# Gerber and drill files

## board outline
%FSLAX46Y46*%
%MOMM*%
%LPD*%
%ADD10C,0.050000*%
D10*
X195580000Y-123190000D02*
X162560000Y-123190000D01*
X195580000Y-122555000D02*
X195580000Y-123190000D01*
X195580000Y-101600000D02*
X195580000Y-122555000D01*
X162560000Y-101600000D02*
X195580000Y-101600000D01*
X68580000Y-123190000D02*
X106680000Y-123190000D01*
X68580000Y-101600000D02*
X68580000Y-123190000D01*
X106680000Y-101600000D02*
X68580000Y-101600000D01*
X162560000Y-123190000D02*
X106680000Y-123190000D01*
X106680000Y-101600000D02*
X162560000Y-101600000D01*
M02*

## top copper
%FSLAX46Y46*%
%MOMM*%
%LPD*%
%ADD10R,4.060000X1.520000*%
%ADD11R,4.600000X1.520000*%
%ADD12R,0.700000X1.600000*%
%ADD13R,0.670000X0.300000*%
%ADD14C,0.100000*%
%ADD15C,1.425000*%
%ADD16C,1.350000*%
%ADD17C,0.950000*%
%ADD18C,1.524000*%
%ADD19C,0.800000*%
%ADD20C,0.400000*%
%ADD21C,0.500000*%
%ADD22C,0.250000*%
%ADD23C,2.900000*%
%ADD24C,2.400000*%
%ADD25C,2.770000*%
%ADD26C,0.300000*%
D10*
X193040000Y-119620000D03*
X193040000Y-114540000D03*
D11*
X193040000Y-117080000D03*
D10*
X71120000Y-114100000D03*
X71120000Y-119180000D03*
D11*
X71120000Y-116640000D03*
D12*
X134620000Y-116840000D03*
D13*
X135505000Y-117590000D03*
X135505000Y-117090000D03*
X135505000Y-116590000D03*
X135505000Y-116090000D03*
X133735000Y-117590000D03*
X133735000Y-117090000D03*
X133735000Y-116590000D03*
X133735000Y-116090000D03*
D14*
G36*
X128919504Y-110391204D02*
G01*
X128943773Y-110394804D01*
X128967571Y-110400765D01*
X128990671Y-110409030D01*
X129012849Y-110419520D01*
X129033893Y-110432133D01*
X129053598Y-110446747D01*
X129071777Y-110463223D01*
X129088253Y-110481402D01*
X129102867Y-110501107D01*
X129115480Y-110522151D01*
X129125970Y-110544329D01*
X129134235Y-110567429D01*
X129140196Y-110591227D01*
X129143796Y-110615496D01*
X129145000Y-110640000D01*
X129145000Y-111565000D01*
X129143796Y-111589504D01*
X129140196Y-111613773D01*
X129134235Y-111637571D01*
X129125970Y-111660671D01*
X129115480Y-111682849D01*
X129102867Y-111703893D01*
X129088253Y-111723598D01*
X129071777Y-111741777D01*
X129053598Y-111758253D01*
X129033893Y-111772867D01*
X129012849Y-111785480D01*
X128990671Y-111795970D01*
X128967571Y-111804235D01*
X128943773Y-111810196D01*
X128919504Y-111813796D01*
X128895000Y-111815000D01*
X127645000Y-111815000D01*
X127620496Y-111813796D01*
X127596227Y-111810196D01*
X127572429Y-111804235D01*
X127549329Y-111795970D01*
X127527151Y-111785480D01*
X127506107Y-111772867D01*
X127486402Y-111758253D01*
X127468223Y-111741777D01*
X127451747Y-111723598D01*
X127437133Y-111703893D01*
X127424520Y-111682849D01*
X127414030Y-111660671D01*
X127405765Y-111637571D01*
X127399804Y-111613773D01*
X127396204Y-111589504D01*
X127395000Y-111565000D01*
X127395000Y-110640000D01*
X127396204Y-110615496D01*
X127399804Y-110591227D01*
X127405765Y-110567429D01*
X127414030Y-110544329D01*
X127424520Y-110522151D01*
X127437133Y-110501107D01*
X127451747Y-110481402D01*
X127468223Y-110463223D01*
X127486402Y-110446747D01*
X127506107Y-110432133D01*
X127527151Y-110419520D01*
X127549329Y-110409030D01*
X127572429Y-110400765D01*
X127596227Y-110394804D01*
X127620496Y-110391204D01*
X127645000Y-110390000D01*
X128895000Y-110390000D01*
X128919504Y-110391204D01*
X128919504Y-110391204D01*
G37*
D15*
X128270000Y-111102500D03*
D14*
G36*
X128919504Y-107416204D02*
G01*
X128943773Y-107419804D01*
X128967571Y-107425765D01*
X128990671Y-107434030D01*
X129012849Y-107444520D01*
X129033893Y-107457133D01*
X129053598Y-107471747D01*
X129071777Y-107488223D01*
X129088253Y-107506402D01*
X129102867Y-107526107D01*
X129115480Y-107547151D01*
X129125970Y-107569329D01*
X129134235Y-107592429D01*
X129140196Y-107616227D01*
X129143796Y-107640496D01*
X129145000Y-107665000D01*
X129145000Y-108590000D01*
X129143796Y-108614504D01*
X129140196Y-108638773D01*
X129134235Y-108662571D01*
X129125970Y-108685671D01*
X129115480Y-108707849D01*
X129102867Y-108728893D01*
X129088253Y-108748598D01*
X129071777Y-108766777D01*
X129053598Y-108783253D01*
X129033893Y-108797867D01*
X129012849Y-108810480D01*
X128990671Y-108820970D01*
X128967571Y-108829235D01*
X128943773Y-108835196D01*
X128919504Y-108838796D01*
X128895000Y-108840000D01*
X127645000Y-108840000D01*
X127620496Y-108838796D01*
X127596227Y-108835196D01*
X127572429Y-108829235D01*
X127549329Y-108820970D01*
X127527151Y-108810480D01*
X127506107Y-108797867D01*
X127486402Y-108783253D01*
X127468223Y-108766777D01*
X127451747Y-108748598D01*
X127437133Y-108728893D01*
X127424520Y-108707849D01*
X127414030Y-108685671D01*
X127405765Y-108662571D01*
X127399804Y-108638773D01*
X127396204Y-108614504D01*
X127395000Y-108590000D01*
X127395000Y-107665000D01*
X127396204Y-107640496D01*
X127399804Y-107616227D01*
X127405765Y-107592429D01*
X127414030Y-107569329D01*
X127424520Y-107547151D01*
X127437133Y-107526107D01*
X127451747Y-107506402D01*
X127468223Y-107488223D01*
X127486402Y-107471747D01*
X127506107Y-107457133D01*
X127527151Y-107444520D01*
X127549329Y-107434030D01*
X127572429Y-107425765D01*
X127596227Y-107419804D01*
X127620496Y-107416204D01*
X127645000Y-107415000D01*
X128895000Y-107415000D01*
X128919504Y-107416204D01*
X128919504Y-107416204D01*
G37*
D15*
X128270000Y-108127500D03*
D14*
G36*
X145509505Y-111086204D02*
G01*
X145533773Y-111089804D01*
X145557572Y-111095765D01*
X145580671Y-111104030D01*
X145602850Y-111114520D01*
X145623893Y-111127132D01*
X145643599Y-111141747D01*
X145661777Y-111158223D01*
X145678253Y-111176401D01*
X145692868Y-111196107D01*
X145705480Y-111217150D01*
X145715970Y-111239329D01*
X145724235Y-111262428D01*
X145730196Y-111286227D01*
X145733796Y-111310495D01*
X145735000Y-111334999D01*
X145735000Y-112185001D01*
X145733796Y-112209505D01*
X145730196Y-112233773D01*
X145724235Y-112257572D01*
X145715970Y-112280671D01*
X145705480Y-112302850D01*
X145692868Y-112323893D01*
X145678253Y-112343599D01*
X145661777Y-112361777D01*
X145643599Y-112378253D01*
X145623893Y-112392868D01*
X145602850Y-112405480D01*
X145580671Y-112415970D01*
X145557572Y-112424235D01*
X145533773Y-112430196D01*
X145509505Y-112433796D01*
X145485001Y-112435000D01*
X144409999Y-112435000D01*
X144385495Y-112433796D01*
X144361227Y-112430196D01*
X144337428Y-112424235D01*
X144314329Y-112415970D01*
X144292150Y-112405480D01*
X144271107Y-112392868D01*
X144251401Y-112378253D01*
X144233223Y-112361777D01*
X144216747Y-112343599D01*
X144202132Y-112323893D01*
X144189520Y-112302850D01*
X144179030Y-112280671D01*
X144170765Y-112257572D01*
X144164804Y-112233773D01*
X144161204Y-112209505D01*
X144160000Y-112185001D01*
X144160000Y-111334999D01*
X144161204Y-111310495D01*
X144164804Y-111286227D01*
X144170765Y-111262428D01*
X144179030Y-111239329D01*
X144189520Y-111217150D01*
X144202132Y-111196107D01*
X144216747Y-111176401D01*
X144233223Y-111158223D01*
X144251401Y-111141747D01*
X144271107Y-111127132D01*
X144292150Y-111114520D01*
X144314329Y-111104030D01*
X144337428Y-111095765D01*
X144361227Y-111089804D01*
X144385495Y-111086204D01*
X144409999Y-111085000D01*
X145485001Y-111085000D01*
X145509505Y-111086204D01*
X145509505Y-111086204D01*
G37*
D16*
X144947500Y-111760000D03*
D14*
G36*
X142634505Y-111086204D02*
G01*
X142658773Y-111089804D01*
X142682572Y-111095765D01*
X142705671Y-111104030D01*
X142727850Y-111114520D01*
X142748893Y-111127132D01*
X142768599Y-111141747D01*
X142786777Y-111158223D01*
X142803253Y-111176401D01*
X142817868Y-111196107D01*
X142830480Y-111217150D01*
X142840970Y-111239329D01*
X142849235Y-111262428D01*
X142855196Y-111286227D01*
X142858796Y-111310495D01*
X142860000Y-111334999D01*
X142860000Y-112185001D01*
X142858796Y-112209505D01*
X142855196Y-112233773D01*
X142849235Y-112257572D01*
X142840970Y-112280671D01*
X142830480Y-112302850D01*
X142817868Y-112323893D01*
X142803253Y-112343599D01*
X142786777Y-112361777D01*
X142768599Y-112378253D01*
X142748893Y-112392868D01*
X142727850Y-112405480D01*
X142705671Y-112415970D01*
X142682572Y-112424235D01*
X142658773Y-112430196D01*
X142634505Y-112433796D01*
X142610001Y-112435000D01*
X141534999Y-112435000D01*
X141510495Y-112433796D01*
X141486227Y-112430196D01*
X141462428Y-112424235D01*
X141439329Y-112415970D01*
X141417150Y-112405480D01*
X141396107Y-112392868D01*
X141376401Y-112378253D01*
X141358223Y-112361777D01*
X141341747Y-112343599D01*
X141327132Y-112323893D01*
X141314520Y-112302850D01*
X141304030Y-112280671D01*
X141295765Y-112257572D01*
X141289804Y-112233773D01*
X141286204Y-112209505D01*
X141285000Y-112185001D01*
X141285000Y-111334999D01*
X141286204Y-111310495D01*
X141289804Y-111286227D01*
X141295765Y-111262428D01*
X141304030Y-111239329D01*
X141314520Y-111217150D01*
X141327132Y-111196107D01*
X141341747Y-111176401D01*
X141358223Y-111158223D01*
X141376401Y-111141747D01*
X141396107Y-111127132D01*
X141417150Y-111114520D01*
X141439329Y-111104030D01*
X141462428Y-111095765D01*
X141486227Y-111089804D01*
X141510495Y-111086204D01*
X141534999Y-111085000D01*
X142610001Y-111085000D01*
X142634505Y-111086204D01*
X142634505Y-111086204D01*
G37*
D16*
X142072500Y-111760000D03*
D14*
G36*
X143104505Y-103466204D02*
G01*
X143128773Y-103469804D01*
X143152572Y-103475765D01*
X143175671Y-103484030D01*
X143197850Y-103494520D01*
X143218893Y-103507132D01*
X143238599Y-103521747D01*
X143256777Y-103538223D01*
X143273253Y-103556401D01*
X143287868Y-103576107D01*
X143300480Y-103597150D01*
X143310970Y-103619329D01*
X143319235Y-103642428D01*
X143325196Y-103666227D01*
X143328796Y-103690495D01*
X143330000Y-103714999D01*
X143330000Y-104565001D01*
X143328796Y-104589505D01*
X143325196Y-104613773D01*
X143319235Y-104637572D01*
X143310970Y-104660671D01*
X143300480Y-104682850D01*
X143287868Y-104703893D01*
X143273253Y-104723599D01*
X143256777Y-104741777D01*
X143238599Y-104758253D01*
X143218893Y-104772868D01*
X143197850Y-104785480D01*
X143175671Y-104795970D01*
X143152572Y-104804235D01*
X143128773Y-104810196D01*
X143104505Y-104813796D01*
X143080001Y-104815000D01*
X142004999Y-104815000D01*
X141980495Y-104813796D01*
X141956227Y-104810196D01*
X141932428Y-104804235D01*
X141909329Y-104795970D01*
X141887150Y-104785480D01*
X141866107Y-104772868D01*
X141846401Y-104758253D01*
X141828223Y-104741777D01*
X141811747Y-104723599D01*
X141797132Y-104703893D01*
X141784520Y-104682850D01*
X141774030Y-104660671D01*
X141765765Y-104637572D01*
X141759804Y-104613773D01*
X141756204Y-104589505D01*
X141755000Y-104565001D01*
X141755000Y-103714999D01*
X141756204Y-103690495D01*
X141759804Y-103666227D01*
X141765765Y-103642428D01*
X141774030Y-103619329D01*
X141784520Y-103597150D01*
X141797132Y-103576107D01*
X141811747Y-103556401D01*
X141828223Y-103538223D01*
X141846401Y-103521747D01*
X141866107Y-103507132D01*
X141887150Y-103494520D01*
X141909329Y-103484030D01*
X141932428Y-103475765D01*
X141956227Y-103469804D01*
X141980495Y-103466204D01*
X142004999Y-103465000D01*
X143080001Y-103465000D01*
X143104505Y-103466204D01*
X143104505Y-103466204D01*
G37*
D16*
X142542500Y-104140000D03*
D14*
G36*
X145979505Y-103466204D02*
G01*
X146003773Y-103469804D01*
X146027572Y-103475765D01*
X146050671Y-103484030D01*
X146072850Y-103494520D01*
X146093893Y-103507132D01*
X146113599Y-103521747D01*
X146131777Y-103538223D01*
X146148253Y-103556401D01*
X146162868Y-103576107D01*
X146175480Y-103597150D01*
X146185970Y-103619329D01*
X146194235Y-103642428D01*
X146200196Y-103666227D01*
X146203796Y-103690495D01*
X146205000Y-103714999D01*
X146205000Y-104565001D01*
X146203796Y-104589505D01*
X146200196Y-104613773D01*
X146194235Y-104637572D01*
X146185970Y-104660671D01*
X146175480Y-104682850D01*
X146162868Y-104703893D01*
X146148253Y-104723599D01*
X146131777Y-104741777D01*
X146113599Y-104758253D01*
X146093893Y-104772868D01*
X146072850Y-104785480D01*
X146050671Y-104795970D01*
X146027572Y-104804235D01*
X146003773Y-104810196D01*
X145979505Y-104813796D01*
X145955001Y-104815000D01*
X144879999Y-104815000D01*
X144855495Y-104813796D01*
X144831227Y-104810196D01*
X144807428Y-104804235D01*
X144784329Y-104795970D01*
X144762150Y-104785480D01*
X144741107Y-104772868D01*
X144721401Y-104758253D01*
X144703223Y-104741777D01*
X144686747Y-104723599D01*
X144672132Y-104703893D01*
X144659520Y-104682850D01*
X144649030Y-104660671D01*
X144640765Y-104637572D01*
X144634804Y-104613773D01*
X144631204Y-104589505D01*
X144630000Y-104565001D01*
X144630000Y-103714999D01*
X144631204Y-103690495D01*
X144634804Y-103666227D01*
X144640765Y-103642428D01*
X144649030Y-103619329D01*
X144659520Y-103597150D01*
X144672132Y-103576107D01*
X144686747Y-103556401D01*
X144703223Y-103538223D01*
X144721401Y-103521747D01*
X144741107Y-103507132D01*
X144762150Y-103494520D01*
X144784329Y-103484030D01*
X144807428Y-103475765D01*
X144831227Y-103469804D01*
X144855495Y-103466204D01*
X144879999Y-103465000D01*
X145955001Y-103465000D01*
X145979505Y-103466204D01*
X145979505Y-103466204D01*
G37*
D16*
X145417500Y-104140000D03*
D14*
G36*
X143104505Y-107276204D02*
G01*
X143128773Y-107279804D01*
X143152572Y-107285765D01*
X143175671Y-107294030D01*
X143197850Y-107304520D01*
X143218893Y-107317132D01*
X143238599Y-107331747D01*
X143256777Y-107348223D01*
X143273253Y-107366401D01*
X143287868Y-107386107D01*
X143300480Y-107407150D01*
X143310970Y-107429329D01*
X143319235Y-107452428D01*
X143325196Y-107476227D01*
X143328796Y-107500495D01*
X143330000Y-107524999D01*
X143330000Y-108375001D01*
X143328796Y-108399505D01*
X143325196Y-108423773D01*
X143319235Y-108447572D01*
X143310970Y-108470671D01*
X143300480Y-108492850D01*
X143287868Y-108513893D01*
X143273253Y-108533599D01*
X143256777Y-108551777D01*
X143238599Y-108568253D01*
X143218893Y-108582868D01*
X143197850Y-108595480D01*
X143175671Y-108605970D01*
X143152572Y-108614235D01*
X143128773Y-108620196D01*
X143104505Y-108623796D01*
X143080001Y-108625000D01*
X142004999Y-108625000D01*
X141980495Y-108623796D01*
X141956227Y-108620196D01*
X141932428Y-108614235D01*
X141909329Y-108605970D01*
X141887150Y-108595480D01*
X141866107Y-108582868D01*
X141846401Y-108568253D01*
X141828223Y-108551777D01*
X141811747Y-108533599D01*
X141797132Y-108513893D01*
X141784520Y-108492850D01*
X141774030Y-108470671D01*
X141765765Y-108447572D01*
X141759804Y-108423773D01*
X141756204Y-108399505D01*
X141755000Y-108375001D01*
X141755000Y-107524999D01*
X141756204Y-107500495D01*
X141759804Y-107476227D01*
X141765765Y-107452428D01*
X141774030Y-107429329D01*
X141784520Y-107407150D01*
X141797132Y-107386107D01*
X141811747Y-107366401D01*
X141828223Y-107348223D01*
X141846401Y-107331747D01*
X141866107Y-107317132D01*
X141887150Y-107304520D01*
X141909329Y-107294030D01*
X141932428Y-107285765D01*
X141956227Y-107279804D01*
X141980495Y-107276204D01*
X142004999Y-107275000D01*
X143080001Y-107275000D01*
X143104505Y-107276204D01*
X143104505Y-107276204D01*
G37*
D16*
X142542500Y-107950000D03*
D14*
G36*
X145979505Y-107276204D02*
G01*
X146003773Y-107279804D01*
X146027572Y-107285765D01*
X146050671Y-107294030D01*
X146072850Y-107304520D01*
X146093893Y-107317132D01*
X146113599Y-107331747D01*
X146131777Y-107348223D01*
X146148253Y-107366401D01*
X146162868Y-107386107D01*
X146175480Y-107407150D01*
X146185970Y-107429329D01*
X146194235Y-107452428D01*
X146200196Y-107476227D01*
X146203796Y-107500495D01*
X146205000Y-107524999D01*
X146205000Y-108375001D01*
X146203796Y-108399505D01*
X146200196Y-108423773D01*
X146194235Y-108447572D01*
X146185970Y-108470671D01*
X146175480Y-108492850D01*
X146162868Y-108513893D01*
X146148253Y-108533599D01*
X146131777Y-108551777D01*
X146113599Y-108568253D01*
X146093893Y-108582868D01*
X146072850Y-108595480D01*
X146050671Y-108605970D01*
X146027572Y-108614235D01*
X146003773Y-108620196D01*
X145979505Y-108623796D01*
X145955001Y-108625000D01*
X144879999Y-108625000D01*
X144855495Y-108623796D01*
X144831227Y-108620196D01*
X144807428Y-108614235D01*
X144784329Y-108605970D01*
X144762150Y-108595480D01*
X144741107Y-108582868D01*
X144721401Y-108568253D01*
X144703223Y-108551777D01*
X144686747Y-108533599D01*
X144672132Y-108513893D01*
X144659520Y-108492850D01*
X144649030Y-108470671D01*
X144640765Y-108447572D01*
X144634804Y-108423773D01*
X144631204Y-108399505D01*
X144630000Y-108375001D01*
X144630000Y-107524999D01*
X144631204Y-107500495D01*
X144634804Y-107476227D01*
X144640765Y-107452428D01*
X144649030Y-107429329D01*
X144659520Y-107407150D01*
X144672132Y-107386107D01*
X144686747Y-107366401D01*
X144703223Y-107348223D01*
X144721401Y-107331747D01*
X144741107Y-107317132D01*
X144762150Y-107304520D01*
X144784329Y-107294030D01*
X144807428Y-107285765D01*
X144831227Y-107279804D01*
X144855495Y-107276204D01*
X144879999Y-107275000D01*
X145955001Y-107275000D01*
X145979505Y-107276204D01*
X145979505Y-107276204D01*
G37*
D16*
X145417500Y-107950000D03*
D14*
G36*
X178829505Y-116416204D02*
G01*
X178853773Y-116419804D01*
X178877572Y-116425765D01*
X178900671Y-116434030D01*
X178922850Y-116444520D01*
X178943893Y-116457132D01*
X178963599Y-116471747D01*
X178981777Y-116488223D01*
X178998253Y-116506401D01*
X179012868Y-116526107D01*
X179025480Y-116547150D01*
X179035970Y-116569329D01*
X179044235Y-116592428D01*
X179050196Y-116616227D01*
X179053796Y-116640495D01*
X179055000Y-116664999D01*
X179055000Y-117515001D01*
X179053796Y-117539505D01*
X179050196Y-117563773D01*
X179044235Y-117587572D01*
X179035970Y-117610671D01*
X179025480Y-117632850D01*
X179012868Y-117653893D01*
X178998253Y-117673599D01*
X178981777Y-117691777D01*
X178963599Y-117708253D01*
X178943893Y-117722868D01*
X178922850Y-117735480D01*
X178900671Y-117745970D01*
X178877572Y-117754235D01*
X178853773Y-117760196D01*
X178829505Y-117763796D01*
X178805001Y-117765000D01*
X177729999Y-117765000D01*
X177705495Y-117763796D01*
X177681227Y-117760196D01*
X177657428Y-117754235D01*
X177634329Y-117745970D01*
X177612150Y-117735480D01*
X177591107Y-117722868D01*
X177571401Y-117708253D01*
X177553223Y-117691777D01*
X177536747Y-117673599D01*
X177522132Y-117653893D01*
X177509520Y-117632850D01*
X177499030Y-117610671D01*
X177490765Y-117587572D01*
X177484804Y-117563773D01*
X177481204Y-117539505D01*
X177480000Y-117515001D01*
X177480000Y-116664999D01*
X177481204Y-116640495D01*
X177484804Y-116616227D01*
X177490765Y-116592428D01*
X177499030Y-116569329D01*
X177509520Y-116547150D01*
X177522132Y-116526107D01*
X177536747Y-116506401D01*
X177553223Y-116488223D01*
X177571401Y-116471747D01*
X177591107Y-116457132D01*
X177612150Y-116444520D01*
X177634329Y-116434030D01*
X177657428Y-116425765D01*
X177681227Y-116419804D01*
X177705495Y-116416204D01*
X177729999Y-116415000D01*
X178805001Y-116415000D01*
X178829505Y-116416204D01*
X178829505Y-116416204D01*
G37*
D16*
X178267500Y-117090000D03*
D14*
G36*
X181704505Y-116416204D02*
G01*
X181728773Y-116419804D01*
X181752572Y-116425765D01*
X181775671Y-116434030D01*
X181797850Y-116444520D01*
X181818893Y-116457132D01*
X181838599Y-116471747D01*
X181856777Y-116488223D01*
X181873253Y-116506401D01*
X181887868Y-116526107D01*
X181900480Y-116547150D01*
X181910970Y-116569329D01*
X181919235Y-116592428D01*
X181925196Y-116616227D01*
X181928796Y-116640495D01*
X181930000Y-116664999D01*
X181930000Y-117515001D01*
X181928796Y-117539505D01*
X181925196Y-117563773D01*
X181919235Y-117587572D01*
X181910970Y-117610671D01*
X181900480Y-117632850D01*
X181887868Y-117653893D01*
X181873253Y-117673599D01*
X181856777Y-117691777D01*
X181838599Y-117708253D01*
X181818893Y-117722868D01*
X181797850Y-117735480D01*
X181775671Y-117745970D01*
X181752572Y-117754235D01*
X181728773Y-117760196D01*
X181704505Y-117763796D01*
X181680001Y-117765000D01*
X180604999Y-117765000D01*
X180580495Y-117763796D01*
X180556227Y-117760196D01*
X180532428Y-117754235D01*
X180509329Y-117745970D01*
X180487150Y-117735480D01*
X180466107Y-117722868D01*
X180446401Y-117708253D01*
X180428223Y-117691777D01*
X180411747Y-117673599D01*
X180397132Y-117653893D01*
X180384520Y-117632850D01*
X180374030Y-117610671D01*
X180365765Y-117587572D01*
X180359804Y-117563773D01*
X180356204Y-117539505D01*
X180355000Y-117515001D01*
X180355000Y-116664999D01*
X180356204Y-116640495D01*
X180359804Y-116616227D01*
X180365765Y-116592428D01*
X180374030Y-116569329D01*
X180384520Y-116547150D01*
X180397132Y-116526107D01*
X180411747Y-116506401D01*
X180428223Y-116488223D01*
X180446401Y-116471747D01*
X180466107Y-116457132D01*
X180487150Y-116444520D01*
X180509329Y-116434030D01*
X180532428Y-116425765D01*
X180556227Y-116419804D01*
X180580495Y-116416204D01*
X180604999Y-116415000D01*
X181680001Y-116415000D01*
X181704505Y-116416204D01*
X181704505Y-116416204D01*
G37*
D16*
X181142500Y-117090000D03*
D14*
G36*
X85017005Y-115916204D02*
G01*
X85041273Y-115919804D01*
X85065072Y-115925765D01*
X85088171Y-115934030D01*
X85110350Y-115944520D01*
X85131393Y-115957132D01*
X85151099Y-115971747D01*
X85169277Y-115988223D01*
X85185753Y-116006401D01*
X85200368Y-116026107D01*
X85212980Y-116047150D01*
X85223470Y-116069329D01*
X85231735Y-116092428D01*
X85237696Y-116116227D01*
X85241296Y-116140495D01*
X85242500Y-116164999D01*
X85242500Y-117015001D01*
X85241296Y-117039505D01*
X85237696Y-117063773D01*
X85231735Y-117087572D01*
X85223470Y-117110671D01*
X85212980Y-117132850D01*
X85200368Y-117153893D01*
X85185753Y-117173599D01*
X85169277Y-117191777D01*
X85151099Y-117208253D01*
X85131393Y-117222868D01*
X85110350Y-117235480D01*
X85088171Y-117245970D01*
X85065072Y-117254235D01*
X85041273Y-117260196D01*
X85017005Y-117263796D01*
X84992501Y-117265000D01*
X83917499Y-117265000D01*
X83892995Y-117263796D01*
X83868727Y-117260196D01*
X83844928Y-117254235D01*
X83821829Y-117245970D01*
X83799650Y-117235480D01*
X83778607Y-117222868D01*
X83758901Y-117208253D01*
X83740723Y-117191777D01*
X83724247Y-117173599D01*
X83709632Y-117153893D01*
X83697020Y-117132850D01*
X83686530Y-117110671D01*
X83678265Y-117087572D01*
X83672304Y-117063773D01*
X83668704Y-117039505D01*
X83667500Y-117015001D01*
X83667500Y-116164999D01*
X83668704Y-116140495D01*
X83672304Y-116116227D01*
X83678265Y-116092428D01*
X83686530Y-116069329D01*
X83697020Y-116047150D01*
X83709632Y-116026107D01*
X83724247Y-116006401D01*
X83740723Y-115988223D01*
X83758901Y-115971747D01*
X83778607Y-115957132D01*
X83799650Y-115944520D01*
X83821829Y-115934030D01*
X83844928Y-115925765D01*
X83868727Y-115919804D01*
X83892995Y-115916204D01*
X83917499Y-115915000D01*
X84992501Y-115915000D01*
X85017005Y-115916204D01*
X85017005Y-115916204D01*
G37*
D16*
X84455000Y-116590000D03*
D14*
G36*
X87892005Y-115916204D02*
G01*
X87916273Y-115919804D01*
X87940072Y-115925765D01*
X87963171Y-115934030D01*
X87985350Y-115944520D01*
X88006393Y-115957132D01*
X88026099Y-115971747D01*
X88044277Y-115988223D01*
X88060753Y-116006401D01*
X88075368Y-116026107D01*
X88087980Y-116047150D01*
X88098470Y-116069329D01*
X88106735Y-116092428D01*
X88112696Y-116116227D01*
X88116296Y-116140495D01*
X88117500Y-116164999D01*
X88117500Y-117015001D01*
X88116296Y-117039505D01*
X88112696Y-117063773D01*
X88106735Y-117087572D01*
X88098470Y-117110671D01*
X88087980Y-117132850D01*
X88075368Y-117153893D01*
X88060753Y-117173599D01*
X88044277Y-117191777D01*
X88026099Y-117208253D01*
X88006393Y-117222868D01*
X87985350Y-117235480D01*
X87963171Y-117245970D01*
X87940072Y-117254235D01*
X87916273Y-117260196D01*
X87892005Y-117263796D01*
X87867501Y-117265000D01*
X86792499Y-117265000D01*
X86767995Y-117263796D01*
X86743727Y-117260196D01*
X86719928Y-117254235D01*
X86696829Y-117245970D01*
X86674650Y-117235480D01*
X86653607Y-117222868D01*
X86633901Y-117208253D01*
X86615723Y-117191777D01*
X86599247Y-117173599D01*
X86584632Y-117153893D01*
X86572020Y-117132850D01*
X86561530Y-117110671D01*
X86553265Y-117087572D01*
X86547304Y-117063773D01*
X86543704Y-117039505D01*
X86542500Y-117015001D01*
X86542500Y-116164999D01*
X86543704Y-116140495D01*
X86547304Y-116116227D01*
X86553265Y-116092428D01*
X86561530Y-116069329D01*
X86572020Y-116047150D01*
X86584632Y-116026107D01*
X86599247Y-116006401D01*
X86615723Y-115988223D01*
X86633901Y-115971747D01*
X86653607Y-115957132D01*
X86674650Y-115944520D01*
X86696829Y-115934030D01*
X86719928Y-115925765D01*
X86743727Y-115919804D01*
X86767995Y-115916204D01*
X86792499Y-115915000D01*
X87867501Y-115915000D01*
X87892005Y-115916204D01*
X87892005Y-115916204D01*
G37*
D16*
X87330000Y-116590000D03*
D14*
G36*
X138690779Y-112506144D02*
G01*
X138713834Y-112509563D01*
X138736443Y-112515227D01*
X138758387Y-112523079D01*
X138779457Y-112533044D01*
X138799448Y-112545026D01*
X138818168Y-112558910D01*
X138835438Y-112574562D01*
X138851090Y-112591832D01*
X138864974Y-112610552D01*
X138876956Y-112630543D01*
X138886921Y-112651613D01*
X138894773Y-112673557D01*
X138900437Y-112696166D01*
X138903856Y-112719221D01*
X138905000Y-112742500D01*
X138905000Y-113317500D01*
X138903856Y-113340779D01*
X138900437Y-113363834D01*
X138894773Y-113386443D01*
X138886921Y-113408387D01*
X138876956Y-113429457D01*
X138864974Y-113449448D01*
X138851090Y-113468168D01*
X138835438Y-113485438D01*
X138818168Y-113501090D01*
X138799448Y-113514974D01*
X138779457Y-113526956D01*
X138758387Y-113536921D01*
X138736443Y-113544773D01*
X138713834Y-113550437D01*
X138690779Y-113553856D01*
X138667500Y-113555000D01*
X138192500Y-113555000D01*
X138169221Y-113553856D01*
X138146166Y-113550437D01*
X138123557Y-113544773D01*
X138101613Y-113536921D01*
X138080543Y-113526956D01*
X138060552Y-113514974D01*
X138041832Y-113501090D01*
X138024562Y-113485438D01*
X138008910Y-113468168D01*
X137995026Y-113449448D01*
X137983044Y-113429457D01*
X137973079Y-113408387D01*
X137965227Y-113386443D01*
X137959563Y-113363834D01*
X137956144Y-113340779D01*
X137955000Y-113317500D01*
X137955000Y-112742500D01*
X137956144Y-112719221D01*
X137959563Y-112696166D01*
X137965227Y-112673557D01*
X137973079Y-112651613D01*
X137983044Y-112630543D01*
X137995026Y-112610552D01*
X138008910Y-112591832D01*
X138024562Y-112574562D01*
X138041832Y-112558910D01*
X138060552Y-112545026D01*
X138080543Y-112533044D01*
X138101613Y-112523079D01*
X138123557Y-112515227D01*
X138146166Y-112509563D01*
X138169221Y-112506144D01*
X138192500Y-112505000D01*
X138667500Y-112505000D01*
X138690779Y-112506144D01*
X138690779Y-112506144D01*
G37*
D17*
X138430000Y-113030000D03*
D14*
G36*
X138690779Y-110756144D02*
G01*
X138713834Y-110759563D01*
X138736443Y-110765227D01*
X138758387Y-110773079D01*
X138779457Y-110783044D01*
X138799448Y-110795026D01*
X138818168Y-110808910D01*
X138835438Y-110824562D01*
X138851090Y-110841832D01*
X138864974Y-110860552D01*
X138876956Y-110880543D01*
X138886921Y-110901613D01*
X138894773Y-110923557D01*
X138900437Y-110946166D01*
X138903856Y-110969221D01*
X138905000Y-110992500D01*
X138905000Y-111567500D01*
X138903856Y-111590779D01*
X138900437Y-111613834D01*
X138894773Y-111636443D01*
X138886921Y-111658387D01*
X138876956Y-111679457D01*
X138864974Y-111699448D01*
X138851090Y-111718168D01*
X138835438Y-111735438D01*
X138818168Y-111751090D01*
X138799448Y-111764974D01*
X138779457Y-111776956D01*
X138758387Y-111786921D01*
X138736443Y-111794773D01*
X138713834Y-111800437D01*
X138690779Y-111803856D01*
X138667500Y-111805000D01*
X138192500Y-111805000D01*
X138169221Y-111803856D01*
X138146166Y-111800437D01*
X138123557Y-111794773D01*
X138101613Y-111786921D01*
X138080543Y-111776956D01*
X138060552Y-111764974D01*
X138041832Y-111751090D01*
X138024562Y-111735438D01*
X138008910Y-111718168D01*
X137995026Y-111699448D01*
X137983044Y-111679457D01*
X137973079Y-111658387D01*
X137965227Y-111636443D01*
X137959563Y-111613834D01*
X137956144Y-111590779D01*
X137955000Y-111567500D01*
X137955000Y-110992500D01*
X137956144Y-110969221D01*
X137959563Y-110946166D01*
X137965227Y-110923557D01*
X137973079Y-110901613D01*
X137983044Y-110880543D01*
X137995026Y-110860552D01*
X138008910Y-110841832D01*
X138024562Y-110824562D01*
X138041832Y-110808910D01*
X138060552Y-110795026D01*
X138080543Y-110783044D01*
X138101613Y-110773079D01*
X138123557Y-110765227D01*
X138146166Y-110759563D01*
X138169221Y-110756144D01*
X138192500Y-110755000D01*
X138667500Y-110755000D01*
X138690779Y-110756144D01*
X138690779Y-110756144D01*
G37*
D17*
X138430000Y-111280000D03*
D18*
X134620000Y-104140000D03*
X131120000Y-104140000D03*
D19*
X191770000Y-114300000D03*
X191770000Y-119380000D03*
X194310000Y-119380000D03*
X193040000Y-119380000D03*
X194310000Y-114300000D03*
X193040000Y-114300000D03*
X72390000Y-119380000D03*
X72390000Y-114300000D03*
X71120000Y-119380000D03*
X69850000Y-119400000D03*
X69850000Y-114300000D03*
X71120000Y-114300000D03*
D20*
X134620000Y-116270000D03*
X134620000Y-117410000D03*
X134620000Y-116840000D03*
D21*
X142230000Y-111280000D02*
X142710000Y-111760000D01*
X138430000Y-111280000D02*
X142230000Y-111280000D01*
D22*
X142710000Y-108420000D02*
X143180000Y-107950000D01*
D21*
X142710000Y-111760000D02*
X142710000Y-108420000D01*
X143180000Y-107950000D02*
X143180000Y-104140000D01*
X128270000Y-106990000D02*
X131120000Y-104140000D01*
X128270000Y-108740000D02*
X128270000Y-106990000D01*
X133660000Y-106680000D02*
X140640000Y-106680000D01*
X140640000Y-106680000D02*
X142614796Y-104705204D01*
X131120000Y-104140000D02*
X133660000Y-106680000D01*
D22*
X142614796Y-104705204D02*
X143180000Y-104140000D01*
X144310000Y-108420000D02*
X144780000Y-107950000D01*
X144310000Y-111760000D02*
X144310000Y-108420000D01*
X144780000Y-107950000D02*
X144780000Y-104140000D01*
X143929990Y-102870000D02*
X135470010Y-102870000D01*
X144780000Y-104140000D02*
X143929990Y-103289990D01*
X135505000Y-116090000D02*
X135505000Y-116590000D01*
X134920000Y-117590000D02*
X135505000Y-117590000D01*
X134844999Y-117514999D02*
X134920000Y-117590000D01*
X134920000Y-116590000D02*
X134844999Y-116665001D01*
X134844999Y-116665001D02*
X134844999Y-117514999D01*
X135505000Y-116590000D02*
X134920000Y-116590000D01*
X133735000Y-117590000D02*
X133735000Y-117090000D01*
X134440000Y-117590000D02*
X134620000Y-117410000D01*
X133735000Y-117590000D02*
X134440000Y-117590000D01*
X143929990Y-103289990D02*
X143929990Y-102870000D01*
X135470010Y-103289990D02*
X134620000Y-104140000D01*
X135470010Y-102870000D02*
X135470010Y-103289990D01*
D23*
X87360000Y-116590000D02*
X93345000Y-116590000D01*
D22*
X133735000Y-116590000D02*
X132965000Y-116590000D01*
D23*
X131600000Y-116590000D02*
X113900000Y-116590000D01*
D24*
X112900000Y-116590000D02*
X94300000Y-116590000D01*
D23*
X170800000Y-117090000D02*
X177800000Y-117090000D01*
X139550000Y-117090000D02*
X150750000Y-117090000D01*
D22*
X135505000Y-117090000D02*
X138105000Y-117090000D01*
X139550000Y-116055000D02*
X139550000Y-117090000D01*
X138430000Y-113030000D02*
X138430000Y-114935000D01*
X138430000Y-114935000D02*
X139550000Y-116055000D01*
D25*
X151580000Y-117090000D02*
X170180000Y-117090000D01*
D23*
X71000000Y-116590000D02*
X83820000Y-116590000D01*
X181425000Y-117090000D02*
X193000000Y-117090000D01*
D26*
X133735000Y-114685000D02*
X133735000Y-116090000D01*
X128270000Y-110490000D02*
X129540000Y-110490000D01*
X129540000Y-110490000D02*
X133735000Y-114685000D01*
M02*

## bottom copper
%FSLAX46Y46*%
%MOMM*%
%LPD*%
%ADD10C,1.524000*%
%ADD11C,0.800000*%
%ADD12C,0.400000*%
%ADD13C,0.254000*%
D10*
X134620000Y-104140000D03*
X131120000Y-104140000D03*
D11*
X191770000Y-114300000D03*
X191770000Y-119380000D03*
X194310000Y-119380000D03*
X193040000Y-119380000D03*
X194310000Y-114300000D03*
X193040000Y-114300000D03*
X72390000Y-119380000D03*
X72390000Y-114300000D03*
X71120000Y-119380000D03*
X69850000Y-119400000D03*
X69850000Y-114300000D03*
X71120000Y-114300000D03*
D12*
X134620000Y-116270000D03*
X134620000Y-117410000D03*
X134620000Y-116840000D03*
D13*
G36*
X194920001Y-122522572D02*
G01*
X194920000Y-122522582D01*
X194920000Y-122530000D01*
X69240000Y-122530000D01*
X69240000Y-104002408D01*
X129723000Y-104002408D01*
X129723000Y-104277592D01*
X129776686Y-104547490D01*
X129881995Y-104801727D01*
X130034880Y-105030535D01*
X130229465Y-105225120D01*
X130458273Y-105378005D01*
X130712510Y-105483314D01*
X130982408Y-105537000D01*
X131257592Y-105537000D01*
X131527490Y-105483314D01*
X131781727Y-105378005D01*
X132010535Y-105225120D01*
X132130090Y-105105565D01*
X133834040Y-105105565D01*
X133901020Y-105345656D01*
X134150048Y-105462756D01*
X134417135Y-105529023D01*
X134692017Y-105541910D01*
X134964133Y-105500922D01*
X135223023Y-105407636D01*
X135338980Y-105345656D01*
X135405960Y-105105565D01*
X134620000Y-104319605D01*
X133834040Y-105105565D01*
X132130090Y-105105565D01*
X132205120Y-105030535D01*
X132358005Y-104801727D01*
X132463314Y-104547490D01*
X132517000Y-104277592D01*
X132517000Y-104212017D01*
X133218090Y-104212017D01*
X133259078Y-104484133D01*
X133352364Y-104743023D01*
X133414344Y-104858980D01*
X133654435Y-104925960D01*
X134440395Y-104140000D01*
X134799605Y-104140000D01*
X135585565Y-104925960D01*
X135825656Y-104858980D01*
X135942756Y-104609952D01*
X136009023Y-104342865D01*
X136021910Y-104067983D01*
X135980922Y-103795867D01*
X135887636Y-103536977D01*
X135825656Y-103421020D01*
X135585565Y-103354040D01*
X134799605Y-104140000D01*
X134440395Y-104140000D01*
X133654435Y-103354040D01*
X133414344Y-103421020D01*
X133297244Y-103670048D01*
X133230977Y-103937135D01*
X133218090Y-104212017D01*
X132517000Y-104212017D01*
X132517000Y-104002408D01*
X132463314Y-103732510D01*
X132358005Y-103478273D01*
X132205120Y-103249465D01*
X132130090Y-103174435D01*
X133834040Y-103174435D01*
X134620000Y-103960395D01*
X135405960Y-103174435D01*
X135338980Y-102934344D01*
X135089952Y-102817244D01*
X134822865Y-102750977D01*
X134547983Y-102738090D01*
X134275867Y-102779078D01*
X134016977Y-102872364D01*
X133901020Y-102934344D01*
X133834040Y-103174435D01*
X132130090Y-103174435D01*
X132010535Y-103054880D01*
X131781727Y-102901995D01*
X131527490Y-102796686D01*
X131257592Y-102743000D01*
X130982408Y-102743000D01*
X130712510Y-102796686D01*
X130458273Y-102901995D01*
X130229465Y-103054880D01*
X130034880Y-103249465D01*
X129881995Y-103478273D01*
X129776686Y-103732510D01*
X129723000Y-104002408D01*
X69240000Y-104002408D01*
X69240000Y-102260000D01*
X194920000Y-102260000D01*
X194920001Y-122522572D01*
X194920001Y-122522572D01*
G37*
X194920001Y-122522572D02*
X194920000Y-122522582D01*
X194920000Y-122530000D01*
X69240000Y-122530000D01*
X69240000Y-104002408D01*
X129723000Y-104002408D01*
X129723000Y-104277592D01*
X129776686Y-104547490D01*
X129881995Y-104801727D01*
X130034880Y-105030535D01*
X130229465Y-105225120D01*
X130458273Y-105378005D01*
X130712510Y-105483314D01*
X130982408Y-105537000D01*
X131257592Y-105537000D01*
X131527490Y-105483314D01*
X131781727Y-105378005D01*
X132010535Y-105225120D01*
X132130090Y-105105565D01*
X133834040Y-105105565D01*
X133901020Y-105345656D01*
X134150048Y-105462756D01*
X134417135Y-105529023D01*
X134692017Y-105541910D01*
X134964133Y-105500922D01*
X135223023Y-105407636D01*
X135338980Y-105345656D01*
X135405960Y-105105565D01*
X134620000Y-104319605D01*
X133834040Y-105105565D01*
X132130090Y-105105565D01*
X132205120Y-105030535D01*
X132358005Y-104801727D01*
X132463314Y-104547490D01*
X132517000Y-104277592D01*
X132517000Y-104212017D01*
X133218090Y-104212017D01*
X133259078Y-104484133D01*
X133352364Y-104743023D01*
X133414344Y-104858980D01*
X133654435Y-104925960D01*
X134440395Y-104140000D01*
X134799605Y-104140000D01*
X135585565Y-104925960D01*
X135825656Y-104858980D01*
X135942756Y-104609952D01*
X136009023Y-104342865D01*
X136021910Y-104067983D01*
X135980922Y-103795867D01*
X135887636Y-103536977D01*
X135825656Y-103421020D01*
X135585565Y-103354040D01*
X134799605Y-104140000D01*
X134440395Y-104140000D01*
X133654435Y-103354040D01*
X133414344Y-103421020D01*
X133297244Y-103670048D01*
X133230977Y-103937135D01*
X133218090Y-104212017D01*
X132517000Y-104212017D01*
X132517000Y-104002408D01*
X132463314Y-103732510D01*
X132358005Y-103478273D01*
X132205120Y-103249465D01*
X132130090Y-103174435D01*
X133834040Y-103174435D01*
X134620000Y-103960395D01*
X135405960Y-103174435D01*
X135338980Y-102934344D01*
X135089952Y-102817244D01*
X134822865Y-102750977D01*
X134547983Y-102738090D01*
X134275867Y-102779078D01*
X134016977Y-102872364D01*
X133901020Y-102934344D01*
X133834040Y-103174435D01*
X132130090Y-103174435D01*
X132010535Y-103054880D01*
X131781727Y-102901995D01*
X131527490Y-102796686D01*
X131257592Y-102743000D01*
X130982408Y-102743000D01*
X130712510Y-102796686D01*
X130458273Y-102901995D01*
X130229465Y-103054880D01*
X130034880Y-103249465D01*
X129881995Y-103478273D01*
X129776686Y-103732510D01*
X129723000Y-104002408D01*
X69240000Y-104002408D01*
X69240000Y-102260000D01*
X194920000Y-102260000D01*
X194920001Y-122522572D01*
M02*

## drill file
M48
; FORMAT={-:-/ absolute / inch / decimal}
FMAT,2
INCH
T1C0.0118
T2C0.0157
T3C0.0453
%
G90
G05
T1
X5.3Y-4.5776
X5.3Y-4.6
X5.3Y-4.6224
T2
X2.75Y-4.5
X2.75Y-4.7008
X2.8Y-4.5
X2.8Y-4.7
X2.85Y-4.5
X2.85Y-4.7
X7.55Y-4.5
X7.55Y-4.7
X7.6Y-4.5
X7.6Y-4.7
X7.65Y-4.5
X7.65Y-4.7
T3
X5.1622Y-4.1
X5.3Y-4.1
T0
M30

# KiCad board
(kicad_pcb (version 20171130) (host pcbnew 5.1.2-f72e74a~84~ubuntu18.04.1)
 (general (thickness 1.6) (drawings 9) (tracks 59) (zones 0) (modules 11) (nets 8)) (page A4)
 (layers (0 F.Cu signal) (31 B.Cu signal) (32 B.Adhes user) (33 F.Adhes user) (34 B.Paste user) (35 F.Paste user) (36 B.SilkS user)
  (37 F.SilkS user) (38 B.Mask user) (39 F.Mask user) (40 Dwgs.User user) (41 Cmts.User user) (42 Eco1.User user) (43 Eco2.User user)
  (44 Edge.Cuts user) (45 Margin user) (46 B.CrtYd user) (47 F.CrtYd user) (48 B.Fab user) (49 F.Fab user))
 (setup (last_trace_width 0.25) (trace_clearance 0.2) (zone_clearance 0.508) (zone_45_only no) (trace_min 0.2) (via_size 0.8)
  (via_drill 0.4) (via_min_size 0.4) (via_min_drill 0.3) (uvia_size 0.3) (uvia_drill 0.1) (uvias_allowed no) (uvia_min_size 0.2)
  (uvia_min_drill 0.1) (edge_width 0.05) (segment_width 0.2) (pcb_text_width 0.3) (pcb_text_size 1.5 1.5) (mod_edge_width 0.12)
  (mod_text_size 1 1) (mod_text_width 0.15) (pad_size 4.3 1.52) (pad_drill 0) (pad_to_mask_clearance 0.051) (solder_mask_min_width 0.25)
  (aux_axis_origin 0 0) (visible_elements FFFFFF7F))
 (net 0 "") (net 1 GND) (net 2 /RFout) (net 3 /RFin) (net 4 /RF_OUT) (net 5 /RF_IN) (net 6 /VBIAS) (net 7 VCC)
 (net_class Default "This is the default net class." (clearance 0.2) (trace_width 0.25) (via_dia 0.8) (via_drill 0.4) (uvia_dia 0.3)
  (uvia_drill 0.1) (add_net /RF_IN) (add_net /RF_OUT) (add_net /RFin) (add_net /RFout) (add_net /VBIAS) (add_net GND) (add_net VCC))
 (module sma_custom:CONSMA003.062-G (layer F.Cu) (at 196.85 119.62)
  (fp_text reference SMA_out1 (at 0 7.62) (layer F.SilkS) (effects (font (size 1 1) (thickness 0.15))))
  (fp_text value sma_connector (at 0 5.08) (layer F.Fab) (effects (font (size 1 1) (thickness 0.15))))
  (pad 3 smd rect (at -3.81 0) (size 4.06 1.52) (layers F.Cu F.Paste F.Mask) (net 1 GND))
  (pad 2 smd rect (at -3.81 -5.08) (size 4.06 1.52) (layers F.Cu F.Paste F.Mask) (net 1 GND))
  (pad 1 smd rect (at -3.81 -2.54) (size 4.6 1.52) (layers F.Cu F.Paste F.Mask) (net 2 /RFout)))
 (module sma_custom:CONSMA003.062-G (layer F.Cu) (at 67.31 114.1 180)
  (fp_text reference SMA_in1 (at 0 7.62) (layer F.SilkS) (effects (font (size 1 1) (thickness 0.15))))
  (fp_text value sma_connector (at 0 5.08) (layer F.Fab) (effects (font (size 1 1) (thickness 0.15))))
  (pad 3 smd rect (at -3.81 0 180) (size 4.06 1.52) (layers F.Cu F.Paste F.Mask) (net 1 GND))
  (pad 2 smd rect (at -3.81 -5.08 180) (size 4.06 1.52) (layers F.Cu F.Paste F.Mask) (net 1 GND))
  (pad 1 smd rect (at -3.81 -2.54 180) (size 4.6 1.52) (layers F.Cu F.Paste F.Mask) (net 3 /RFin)))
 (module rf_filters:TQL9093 (layer F.Cu) (at 134.62 116.84)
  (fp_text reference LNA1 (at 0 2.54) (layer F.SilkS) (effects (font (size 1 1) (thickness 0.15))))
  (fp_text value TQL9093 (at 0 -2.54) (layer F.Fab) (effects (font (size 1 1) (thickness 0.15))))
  (pad 9 smd rect (at 0 0) (size 0.7 1.6) (layers F.Cu F.Paste F.Mask) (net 1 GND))
  (pad 8 smd rect (at 0.885 0.75) (size 0.67 0.3) (layers F.Cu F.Paste F.Mask) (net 1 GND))
  (pad 7 smd rect (at 0.885 0.25) (size 0.67 0.3) (layers F.Cu F.Paste F.Mask) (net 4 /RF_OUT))
  (pad 6 smd rect (at 0.885 -0.25) (size 0.67 0.3) (layers F.Cu F.Paste F.Mask) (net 1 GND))
  (pad 5 smd rect (at 0.885 -0.75) (size 0.67 0.3) (layers F.Cu F.Paste F.Mask) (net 1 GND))
  (pad 4 smd rect (at -0.885 0.75) (size 0.67 0.3) (layers F.Cu F.Paste F.Mask) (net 1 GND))
  (pad 3 smd rect (at -0.885 0.25) (size 0.67 0.3) (layers F.Cu F.Paste F.Mask) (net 1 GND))
  (pad 2 smd rect (at -0.885 -0.25) (size 0.67 0.3) (layers F.Cu F.Paste F.Mask) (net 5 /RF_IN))
  (pad 1 smd rect (at -0.885 -0.75) (size 0.67 0.3) (layers F.Cu F.Paste F.Mask) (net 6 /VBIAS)))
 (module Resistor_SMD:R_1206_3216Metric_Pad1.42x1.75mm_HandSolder (layer F.Cu) (at 128.27 109.615 270)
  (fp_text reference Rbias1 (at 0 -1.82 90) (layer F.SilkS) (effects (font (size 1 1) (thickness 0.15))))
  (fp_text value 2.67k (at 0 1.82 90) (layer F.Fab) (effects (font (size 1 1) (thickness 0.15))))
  (pad 2 smd roundrect (at 1.4875 0 270) (size 1.425 1.75) (layers F.Cu F.Paste F.Mask) (roundrect_rratio 0.175439) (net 6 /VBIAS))
  (pad 1 smd roundrect (at -1.4875 0 270) (size 1.425 1.75) (layers F.Cu F.Paste F.Mask) (roundrect_rratio 0.175439) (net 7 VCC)))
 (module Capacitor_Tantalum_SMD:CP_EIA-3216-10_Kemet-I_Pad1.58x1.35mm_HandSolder (layer F.Cu) (at 143.51 111.76)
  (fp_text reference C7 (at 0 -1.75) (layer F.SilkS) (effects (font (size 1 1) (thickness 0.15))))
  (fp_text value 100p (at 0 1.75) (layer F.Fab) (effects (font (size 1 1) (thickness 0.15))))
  (pad 2 smd roundrect (at 1.4375 0) (size 1.575 1.35) (layers F.Cu F.Paste F.Mask) (roundrect_rratio 0.185185) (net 1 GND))
  (pad 1 smd roundrect (at -1.4375 0) (size 1.575 1.35) (layers F.Cu F.Paste F.Mask) (roundrect_rratio 0.185185) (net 7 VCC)))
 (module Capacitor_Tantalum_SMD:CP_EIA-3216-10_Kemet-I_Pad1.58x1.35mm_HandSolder (layer F.Cu) (at 143.98 104.14 180)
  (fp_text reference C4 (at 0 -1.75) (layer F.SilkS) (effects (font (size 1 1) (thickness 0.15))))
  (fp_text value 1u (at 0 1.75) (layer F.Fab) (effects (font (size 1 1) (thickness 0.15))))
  (pad 2 smd roundrect (at 1.4375 0 180) (size 1.575 1.35) (layers F.Cu F.Paste F.Mask) (roundrect_rratio 0.185185) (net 7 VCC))
  (pad 1 smd roundrect (at -1.4375 0 180) (size 1.575 1.35) (layers F.Cu F.Paste F.Mask) (roundrect_rratio 0.185185) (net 1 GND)))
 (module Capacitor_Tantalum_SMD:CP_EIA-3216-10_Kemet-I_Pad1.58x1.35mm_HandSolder (layer F.Cu) (at 143.98 107.95 180)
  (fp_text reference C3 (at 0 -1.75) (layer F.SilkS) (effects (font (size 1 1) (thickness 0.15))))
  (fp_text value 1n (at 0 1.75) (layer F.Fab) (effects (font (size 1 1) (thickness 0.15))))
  (pad 2 smd roundrect (at 1.4375 0 180) (size 1.575 1.35) (layers F.Cu F.Paste F.Mask) (roundrect_rratio 0.185185) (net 7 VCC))
  (pad 1 smd roundrect (at -1.4375 0 180) (size 1.575 1.35) (layers F.Cu F.Paste F.Mask) (roundrect_rratio 0.185185) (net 1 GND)))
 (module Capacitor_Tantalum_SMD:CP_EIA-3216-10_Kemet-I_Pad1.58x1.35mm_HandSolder (layer F.Cu) (at 179.705 117.09 180)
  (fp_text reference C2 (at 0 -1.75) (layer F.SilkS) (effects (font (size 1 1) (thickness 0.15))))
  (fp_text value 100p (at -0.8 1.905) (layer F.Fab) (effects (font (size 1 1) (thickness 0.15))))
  (pad 2 smd roundrect (at 1.4375 0 180) (size 1.575 1.35) (layers F.Cu F.Paste F.Mask) (roundrect_rratio 0.185185) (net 4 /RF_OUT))
  (pad 1 smd roundrect (at -1.4375 0 180) (size 1.575 1.35) (layers F.Cu F.Paste F.Mask) (roundrect_rratio 0.185185) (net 2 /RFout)))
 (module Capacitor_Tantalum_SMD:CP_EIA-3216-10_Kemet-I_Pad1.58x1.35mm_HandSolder (layer F.Cu) (at 85.8925 116.59 180)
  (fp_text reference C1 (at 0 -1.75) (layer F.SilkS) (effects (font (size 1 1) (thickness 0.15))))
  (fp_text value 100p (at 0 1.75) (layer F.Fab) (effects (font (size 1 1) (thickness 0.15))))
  (pad 2 smd roundrect (at 1.4375 0 180) (size 1.575 1.35) (layers F.Cu F.Paste F.Mask) (roundrect_rratio 0.185185) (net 3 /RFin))
  (pad 1 smd roundrect (at -1.4375 0 180) (size 1.575 1.35) (layers F.Cu F.Paste F.Mask) (roundrect_rratio 0.185185) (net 5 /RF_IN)))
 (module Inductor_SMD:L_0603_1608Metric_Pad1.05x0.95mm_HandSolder (layer F.Cu) (at 138.43 112.155 270)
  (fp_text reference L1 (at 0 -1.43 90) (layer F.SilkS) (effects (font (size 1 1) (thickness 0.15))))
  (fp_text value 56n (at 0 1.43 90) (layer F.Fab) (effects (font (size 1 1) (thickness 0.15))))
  (pad 2 smd roundrect (at 0.875 0 270) (size 1.05 0.95) (layers F.Cu F.Paste F.Mask) (roundrect_rratio 0.25) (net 4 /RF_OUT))
  (pad 1 smd roundrect (at -0.875 0 270) (size 1.05 0.95) (layers F.Cu F.Paste F.Mask) (roundrect_rratio 0.25) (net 7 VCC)))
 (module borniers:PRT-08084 (layer F.Cu) (at 134.62 109.22)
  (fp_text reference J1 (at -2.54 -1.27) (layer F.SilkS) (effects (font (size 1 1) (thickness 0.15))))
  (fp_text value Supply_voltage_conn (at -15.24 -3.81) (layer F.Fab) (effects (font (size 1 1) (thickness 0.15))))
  (pad 2 thru_hole circle (at 0 -5.08) (size 1.524 1.524) (drill 1.15) (layers *.Cu *.Mask) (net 1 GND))
  (pad 1 thru_hole circle (at -3.5 -5.08) (size 1.524 1.524) (drill 1.15) (layers *.Cu *.Mask) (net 7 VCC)))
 (gr_line (start 195.58 123.19) (end 162.56 123.19) (layer Edge.Cuts) (width 0.05))
 (gr_line (start 195.58 122.555) (end 195.58 123.19) (layer Edge.Cuts) (width 0.05))
 (gr_line (start 195.58 101.6) (end 195.58 122.555) (layer Edge.Cuts) (width 0.05))
 (gr_line (start 162.56 101.6) (end 195.58 101.6) (layer Edge.Cuts) (width 0.05))
 (gr_line (start 68.58 123.19) (end 106.68 123.19) (layer Edge.Cuts) (width 0.05))
 (gr_line (start 68.58 101.6) (end 68.58 123.19) (layer Edge.Cuts) (width 0.05))
 (gr_line (start 106.68 101.6) (end 68.58 101.6) (layer Edge.Cuts) (width 0.05))
 (gr_line (start 162.56 123.19) (end 106.68 123.19) (layer Edge.Cuts) (width 0.05))
 (gr_line (start 106.68 101.6) (end 162.56 101.6) (layer Edge.Cuts) (width 0.05))
 (segment (start 142.23 111.28) (end 142.71 111.76) (width 0.5) (layer F.Cu) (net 7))
 (segment (start 138.43 111.28) (end 142.23 111.28) (width 0.5) (layer F.Cu) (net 7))
 (segment (start 142.71 108.42) (end 143.18 107.95) (width 0.25) (layer F.Cu) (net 7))
 (segment (start 142.71 111.76) (end 142.71 108.42) (width 0.5) (layer F.Cu) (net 7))
 (segment (start 143.18 107.95) (end 143.18 104.14) (width 0.5) (layer F.Cu) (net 7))
 (segment (start 128.27 106.99) (end 131.12 104.14) (width 0.5) (layer F.Cu) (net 7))
 (segment (start 128.27 108.74) (end 128.27 106.99) (width 0.5) (layer F.Cu) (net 7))
 (segment (start 133.66 106.68) (end 140.64 106.68) (width 0.5) (layer F.Cu) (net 7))
 (segment (start 140.64 106.68) (end 142.614796 104.705204) (width 0.5) (layer F.Cu) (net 7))
 (segment (start 131.12 104.14) (end 133.66 106.68) (width 0.5) (layer F.Cu) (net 7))
 (segment (start 142.614796 104.705204) (end 143.18 104.14) (width 0.25) (layer F.Cu) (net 7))
 (via (at 191.77 114.3) (size 0.8) (drill 0.4) (layers F.Cu B.Cu) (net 1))
 (via (at 191.77 119.38) (size 0.8) (drill 0.4) (layers F.Cu B.Cu) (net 1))
 (via (at 194.31 119.38) (size 0.8) (drill 0.4) (layers F.Cu B.Cu) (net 1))
 (via (at 193.04 119.38) (size 0.8) (drill 0.4) (layers F.Cu B.Cu) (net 1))
 (via (at 194.31 114.3) (size 0.8) (drill 0.4) (layers F.Cu B.Cu) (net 1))
 (via (at 193.04 114.3) (size 0.8) (drill 0.4) (layers F.Cu B.Cu) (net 1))
 (via (at 72.39 119.38) (size 0.8) (drill 0.4) (layers F.Cu B.Cu) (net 1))
 (via (at 72.39 114.3) (size 0.8) (drill 0.4) (layers F.Cu B.Cu) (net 1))
 (via (at 71.12 119.38) (size 0.8) (drill 0.4) (layers F.Cu B.Cu) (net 1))
 (via (at 69.85 119.4) (size 0.8) (drill 0.4) (layers F.Cu B.Cu) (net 1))
 (via (at 69.85 114.3) (size 0.8) (drill 0.4) (layers F.Cu B.Cu) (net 1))
 (via (at 71.12 114.3) (size 0.8) (drill 0.4) (layers F.Cu B.Cu) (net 1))
 (via (at 134.62 116.27) (size 0.4) (drill 0.3) (layers F.Cu B.Cu) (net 1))
 (via (at 134.62 117.41) (size 0.4) (drill 0.3) (layers F.Cu B.Cu) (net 1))
 (via (at 134.62 116.84) (size 0.4) (drill 0.3) (layers F.Cu B.Cu) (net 1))
 (segment (start 144.31 108.42) (end 144.78 107.95) (width 0.25) (layer F.Cu) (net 1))
 (segment (start 144.31 111.76) (end 144.31 108.42) (width 0.25) (layer F.Cu) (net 1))
 (segment (start 144.78 107.95) (end 144.78 104.14) (width 0.25) (layer F.Cu) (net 1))
 (segment (start 143.92999 102.87) (end 135.47001 102.87) (width 0.25) (layer F.Cu) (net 1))
 (segment (start 144.78 104.14) (end 143.92999 103.28999) (width 0.25) (layer F.Cu) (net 1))
 (segment (start 135.505 116.09) (end 135.505 116.59) (width 0.25) (layer F.Cu) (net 1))
 (segment (start 134.92 117.59) (end 135.505 117.59) (width 0.25) (layer F.Cu) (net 1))
 (segment (start 134.844999 117.514999) (end 134.92 117.59) (width 0.25) (layer F.Cu) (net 1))
 (segment (start 134.92 116.59) (end 134.844999 116.665001) (width 0.25) (layer F.Cu) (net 1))
 (segment (start 134.844999 116.665001) (end 134.844999 117.514999) (width 0.25) (layer F.Cu) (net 1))
 (segment (start 135.505 116.59) (end 134.92 116.59) (width 0.25) (layer F.Cu) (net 1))
 (segment (start 133.735 117.59) (end 133.735 117.09) (width 0.25) (layer F.Cu) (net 1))
 (segment (start 134.44 117.59) (end 134.62 117.41) (width 0.25) (layer F.Cu) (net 1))
 (segment (start 133.735 117.59) (end 134.44 117.59) (width 0.25) (layer F.Cu) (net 1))
 (segment (start 143.92999 103.28999) (end 143.92999 102.87) (width 0.25) (layer F.Cu) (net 1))
 (segment (start 135.47001 103.28999) (end 134.62 104.14) (width 0.25) (layer F.Cu) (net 1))
 (segment (start 135.47001 102.87) (end 135.47001 103.28999) (width 0.25) (layer F.Cu) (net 1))
 (segment (start 87.36 116.59) (end 93.345 116.59) (width 2.9) (layer F.Cu) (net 5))
 (segment (start 133.735 116.59) (end 132.965 116.59) (width 0.25) (layer F.Cu) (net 5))
 (segment (start 131.6 116.59) (end 113.9 116.59) (width 2.9) (layer F.Cu) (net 5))
 (segment (start 112.9 116.59) (end 94.3 116.59) (width 2.4) (layer F.Cu) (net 5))
 (segment (start 170.8 117.09) (end 177.8 117.09) (width 2.9) (layer F.Cu) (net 4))
 (segment (start 139.55 117.09) (end 150.75 117.09) (width 2.9) (layer F.Cu) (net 4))
 (segment (start 135.505 117.09) (end 138.105 117.09) (width 0.25) (layer F.Cu) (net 4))
 (segment (start 139.55 116.055) (end 139.55 117.09) (width 0.25) (layer F.Cu) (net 4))
 (segment (start 138.43 113.03) (end 138.43 114.935) (width 0.25) (layer F.Cu) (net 4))
 (segment (start 138.43 114.935) (end 139.55 116.055) (width 0.25) (layer F.Cu) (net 4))
 (segment (start 151.58 117.09) (end 170.18 117.09) (width 2.77) (layer F.Cu) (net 4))
 (segment (start 71 116.59) (end 83.82 116.59) (width 2.9) (layer F.Cu) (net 3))
 (segment (start 181.425 117.09) (end 193 117.09) (width 2.9) (layer F.Cu) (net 2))
 (segment (start 133.735 114.685) (end 133.735 116.09) (width 0.3) (layer F.Cu) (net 6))
 (segment (start 128.27 110.49) (end 129.54 110.49) (width 0.3) (layer F.Cu) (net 6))
 (segment (start 129.54 110.49) (end 133.735 114.685) (width 0.3) (layer F.Cu) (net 6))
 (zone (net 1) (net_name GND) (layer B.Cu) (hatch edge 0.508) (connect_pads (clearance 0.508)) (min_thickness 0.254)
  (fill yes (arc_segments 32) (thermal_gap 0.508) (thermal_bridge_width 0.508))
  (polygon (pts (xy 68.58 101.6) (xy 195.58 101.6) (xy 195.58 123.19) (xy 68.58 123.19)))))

